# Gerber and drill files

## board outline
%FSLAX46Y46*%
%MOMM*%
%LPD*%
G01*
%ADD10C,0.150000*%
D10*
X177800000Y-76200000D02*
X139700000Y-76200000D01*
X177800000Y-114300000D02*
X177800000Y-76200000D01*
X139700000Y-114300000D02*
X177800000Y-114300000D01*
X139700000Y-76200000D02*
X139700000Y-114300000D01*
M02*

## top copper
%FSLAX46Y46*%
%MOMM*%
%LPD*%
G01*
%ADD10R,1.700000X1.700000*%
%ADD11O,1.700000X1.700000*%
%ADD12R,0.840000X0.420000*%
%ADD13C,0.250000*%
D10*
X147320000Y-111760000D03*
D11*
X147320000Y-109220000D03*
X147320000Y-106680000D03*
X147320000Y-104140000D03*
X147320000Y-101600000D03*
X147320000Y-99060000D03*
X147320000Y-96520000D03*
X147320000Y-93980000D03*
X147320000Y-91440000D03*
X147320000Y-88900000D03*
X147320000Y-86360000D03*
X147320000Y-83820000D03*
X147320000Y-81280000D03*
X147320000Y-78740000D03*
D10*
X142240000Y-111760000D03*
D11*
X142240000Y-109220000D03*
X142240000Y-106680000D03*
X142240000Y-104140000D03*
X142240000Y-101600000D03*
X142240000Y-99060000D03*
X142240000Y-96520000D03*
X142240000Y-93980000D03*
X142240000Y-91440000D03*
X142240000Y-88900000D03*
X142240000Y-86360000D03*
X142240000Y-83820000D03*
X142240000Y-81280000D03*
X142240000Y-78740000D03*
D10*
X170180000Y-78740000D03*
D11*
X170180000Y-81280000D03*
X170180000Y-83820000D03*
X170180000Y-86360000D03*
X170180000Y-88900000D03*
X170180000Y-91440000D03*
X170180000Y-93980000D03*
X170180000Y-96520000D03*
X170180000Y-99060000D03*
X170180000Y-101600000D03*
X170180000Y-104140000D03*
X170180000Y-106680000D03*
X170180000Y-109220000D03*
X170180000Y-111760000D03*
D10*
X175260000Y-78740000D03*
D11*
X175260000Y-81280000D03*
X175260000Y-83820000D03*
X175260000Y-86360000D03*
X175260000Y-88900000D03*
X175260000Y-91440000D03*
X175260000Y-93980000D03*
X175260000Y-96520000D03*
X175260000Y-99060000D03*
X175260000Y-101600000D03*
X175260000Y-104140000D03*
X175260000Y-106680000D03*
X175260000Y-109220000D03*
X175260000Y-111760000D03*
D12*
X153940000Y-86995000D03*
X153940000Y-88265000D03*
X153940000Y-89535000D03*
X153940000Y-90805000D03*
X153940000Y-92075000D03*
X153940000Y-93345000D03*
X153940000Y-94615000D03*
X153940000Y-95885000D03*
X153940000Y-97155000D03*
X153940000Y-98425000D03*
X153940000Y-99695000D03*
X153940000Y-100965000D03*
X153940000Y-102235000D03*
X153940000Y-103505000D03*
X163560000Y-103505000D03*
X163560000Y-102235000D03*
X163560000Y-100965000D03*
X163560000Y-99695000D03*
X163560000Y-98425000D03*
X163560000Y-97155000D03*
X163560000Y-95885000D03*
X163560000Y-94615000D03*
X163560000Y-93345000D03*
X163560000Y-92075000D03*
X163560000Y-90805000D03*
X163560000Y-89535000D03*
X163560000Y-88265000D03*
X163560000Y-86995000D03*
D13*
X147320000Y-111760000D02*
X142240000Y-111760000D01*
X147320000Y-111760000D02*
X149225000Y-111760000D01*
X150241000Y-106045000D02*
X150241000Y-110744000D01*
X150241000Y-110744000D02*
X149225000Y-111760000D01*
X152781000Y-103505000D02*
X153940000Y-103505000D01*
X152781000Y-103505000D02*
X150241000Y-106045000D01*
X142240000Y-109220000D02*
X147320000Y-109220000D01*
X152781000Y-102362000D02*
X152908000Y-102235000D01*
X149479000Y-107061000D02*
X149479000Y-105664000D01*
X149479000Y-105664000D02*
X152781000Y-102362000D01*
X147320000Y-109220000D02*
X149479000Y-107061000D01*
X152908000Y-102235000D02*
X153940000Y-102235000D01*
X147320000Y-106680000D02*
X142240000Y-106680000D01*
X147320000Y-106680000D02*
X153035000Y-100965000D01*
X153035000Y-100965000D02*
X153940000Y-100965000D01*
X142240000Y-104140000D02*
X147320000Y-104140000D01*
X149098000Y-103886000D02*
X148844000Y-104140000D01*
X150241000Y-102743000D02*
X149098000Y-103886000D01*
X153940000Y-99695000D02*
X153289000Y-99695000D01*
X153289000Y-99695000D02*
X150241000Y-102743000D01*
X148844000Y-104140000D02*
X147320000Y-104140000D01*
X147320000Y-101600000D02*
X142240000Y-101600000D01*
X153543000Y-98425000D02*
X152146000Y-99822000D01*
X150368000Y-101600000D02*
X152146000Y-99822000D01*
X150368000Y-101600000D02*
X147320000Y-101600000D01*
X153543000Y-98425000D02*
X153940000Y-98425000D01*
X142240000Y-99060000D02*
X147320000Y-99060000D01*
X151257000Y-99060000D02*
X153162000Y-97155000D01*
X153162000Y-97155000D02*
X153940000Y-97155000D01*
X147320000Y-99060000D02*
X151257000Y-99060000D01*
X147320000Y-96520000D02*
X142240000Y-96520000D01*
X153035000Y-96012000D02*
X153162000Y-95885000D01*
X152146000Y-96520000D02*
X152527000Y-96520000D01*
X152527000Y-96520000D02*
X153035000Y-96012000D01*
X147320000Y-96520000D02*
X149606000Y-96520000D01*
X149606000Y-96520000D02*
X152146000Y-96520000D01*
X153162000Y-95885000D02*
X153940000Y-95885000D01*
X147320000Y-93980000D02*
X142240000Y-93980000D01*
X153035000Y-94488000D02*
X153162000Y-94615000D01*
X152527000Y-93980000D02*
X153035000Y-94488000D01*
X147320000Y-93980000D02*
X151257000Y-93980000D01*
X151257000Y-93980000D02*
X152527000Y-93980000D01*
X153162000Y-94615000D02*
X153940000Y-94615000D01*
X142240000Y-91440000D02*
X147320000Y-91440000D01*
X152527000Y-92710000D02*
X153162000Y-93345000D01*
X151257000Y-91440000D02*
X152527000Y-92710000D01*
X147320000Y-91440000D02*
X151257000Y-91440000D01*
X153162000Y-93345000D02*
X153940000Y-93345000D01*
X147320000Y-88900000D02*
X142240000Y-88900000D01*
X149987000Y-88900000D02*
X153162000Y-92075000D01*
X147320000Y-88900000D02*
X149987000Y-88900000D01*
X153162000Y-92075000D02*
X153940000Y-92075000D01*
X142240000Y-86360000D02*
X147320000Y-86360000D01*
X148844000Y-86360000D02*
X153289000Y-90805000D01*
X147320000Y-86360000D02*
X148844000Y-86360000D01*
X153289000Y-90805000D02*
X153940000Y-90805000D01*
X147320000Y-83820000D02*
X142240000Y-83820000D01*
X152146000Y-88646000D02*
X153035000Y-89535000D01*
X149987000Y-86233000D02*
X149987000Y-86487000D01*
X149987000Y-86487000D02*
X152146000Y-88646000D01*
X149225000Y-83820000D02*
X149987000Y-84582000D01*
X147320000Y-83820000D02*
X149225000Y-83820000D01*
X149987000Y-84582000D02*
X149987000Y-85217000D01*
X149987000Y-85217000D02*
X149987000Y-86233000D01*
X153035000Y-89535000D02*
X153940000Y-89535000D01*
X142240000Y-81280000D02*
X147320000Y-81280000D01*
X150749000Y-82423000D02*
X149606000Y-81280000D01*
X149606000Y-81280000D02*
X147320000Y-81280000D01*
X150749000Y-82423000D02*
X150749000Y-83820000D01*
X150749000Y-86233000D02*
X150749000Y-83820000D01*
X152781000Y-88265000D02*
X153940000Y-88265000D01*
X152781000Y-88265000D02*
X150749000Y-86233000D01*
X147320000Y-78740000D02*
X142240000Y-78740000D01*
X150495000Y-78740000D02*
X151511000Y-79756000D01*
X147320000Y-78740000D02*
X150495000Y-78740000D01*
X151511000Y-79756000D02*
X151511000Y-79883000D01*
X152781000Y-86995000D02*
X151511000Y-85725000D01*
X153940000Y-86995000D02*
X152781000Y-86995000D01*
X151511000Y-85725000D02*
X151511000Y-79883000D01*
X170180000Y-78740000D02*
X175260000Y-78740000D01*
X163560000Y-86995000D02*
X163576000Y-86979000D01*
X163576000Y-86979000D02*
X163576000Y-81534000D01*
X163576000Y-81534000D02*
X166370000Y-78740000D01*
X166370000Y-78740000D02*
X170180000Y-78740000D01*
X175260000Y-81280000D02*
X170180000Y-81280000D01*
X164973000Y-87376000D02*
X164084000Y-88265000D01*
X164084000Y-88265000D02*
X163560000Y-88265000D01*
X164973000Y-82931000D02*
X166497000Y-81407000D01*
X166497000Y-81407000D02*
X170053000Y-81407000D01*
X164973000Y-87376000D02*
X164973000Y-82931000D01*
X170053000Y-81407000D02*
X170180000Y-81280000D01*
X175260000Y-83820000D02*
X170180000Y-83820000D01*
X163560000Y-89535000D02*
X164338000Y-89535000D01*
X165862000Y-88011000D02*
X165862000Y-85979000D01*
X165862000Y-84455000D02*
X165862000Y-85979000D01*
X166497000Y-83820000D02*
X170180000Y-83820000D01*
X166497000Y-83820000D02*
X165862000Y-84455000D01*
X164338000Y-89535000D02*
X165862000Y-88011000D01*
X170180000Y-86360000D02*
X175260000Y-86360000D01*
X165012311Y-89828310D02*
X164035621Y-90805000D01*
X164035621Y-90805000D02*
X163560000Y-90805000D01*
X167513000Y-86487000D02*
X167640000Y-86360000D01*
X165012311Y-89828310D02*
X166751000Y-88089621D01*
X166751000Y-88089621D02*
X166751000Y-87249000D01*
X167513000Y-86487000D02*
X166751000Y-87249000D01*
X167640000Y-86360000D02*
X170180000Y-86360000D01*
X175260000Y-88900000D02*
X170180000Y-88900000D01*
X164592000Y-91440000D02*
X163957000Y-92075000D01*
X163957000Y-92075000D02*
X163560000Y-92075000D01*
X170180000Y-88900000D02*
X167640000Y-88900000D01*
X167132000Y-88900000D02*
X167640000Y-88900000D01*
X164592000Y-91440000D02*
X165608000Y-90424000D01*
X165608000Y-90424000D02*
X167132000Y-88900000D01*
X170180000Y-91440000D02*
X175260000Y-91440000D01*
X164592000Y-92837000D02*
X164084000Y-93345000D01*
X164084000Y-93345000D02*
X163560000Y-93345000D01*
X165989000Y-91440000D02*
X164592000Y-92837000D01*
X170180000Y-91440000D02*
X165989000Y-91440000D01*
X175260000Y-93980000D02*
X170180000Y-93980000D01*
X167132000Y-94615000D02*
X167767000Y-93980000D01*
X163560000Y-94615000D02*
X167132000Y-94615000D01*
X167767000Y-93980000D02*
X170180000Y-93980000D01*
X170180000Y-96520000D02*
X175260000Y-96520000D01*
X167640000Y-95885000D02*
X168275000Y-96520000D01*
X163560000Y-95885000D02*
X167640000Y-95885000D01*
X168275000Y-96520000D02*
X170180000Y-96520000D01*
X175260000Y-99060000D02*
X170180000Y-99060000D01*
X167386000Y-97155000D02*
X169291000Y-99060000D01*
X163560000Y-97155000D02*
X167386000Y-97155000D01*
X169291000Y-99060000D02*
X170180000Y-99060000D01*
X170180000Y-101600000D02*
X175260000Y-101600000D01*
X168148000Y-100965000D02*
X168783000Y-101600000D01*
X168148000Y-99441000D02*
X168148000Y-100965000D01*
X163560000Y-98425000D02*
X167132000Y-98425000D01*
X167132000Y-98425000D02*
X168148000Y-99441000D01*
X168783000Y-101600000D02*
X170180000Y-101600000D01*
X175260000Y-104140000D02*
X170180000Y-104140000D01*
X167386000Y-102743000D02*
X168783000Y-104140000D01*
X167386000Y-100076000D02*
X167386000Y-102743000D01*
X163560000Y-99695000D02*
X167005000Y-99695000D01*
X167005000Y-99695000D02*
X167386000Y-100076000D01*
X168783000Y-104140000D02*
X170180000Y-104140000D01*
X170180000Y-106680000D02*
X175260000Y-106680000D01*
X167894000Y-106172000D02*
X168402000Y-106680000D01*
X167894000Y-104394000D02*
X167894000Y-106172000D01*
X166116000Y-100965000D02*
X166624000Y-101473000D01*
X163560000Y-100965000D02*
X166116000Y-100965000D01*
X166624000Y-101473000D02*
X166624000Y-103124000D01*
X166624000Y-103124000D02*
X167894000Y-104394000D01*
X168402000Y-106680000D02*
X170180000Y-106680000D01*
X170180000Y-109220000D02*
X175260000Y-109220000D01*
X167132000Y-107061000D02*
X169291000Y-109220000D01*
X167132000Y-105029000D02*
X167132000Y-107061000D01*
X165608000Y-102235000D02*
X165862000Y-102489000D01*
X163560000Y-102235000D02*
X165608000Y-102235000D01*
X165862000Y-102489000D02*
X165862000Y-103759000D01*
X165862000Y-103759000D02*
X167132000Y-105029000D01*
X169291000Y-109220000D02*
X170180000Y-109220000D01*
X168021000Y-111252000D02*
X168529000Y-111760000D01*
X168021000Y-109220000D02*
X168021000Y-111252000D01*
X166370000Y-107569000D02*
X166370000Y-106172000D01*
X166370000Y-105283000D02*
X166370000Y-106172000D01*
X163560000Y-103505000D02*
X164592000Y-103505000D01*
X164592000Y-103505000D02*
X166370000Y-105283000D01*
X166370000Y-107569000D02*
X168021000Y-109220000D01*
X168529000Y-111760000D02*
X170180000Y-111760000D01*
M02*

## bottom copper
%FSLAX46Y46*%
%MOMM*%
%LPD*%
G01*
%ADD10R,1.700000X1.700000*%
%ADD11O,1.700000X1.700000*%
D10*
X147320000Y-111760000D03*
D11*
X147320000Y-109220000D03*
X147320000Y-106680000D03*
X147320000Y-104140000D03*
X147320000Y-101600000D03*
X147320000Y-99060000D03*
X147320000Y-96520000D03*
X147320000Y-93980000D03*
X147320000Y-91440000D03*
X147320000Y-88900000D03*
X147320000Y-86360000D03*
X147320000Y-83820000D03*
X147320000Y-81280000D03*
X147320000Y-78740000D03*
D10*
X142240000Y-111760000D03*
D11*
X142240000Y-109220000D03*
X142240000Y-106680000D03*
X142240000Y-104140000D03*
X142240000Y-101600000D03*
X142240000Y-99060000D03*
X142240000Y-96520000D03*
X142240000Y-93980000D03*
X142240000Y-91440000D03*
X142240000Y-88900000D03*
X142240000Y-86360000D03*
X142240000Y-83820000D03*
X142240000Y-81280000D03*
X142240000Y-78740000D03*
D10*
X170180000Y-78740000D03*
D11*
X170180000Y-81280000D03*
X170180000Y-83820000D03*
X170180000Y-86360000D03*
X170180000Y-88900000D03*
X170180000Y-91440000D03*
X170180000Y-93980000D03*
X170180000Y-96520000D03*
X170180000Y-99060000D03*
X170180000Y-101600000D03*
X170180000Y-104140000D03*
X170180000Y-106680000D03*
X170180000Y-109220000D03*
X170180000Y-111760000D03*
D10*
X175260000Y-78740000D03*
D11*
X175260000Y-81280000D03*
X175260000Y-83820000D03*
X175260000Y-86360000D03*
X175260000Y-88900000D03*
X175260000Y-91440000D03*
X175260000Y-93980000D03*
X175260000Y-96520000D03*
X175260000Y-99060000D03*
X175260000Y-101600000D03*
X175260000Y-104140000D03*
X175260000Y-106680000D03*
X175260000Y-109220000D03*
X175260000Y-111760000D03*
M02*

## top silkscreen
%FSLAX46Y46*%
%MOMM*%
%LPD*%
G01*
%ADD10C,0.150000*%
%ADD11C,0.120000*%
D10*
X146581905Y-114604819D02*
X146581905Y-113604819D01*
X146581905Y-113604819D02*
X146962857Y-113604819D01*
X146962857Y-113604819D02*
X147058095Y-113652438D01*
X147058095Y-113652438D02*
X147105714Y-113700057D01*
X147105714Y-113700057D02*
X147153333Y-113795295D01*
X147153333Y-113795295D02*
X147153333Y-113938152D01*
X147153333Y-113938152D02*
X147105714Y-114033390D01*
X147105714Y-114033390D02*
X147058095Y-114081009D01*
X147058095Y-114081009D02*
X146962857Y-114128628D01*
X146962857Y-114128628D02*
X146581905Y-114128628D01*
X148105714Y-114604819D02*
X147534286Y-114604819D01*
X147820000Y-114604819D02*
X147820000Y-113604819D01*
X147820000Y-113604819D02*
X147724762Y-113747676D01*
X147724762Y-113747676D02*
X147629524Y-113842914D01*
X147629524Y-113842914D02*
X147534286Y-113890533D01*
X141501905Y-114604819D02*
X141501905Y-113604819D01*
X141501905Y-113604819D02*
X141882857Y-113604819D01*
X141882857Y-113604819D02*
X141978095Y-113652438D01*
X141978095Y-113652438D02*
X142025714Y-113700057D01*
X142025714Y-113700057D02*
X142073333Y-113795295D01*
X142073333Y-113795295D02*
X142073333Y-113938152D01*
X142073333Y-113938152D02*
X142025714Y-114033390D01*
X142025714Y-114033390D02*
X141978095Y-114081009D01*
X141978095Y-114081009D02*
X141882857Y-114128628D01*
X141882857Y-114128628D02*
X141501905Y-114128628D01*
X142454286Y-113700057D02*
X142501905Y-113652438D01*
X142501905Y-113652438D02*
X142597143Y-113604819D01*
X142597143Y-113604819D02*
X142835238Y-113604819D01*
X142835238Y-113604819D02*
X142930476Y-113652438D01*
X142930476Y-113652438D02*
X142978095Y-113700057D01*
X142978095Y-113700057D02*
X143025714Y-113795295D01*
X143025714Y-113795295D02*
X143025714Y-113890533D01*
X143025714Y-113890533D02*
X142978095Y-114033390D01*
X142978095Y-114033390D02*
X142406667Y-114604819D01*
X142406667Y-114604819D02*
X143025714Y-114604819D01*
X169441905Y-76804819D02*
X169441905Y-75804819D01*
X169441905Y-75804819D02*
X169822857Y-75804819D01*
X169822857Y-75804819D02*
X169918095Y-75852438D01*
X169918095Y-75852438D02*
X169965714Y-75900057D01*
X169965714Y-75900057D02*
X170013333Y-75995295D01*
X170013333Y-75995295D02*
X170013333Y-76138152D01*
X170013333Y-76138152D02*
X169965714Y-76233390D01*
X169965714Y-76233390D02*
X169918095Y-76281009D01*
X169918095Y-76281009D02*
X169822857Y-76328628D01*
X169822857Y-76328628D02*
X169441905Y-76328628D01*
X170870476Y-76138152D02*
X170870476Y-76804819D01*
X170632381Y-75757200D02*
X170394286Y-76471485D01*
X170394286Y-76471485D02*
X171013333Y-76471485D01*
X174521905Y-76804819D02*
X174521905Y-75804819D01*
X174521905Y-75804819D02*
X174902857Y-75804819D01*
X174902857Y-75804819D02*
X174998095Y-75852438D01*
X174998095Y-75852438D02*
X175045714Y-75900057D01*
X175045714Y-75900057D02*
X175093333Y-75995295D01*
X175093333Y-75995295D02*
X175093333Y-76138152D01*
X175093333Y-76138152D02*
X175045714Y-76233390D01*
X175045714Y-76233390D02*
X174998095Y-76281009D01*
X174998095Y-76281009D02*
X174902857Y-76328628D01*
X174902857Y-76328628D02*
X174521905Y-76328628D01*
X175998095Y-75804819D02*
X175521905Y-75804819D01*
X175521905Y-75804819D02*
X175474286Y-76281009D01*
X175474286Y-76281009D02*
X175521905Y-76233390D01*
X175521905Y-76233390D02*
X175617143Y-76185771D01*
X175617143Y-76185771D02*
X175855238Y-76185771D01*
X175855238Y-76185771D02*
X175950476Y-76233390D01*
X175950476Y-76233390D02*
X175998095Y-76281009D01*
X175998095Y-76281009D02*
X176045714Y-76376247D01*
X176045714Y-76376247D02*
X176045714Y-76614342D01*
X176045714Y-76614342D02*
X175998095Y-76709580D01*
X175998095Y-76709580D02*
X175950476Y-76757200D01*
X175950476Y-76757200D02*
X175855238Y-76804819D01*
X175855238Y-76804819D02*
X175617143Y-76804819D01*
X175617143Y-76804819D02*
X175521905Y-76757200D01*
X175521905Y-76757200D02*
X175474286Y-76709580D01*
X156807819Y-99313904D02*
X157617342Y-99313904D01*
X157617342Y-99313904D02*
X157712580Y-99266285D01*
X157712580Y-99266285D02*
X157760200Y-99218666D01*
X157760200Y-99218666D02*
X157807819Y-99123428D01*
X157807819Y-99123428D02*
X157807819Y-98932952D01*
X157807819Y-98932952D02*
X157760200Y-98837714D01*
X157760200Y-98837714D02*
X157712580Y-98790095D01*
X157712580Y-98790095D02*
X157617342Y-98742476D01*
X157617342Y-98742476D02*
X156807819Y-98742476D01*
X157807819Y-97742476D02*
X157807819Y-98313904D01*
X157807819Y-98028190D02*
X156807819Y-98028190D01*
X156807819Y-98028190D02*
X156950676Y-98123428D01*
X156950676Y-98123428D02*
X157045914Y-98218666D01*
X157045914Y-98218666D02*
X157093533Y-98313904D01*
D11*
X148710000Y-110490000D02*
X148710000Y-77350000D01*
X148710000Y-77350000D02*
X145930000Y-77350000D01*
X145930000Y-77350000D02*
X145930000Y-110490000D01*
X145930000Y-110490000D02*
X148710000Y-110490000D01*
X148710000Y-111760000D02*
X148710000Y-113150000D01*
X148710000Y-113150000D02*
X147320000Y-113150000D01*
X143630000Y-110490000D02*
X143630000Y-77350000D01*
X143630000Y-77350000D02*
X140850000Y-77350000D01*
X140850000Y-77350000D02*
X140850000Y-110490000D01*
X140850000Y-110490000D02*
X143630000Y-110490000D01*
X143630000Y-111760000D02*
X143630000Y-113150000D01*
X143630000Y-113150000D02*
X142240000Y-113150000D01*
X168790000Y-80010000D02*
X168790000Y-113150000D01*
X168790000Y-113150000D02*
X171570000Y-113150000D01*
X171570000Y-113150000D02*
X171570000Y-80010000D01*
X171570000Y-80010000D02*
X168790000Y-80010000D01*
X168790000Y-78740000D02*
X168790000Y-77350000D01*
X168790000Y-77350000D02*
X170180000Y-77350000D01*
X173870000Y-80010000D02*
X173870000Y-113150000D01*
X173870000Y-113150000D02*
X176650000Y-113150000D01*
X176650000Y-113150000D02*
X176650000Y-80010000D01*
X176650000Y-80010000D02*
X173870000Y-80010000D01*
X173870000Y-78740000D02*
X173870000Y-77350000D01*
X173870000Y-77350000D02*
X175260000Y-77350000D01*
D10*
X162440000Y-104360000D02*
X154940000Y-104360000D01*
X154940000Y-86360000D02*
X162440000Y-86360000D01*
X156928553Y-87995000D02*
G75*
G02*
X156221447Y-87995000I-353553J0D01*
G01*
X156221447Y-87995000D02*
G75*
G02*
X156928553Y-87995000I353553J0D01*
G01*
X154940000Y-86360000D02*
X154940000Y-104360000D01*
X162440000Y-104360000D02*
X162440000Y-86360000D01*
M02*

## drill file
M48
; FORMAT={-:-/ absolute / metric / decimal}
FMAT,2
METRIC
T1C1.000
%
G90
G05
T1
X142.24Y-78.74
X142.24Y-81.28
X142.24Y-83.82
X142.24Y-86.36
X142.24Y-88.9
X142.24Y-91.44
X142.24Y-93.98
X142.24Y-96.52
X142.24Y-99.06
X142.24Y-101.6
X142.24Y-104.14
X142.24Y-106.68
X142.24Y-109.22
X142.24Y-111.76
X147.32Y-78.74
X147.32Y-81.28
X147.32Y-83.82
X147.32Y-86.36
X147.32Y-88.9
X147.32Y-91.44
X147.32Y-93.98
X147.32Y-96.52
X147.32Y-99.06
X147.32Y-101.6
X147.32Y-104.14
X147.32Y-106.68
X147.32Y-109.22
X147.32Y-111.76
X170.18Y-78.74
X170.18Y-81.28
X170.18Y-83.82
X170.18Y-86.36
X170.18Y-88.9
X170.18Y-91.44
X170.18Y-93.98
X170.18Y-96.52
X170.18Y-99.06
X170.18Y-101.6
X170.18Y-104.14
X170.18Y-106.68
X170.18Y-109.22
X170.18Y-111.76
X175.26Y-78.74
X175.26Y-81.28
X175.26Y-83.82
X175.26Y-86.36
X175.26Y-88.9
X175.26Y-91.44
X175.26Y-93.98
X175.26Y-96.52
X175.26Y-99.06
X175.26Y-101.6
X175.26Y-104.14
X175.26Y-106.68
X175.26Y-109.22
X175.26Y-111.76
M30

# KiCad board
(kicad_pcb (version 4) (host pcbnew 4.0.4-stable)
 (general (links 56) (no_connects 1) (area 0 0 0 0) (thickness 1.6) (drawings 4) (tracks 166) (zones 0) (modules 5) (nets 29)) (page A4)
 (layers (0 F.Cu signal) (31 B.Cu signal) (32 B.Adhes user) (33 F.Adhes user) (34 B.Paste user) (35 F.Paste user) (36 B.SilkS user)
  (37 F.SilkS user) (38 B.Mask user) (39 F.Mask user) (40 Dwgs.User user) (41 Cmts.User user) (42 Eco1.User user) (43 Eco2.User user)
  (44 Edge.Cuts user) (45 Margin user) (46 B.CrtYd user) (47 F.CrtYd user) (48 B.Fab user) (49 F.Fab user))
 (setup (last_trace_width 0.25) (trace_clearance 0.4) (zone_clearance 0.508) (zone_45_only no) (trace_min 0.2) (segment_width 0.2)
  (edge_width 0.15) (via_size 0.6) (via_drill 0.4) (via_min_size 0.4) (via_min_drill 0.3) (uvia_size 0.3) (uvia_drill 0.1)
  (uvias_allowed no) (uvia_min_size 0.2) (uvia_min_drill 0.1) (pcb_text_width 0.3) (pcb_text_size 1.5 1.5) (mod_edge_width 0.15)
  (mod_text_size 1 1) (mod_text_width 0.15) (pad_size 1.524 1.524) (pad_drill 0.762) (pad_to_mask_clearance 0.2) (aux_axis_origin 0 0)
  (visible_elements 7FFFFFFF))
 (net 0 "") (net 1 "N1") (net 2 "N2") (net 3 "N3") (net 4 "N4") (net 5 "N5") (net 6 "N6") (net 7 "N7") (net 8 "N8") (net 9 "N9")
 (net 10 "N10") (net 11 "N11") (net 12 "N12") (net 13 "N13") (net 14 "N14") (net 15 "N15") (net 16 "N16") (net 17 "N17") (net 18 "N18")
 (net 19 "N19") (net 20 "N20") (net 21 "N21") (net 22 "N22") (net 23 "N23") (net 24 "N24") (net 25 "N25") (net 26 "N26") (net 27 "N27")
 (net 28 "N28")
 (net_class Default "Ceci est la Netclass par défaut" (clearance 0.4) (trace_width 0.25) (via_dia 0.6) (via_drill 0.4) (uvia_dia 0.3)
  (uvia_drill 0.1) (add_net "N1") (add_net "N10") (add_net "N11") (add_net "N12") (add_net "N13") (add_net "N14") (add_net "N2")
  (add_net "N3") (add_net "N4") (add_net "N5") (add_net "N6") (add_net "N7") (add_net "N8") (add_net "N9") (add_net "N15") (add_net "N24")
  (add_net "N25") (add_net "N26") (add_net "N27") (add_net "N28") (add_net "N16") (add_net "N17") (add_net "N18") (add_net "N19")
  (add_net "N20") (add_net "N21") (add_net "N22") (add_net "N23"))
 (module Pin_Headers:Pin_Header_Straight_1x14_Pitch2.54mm (layer F.Cu) (at 147.32 111.76 180)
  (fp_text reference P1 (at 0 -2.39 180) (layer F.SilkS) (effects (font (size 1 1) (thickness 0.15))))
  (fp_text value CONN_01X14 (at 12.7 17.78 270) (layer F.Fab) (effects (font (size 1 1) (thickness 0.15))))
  (fp_line (start -1.39 1.27) (end -1.39 34.41) (layer F.SilkS) (width 0.12))
  (fp_line (start -1.39 34.41) (end 1.39 34.41) (layer F.SilkS) (width 0.12))
  (fp_line (start 1.39 34.41) (end 1.39 1.27) (layer F.SilkS) (width 0.12))
  (fp_line (start 1.39 1.27) (end -1.39 1.27) (layer F.SilkS) (width 0.12))
  (fp_line (start -1.39 0) (end -1.39 -1.39) (layer F.SilkS) (width 0.12))
  (fp_line (start -1.39 -1.39) (end 0 -1.39) (layer F.SilkS) (width 0.12))
  (pad 1 thru_hole rect (at 0 0 180) (size 1.7 1.7) (drill 1) (layers *.Cu *.Mask) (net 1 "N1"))
  (pad 2 thru_hole oval (at 0 2.54 180) (size 1.7 1.7) (drill 1) (layers *.Cu *.Mask) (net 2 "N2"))
  (pad 3 thru_hole oval (at 0 5.08 180) (size 1.7 1.7) (drill 1) (layers *.Cu *.Mask) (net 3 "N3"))
  (pad 4 thru_hole oval (at 0 7.62 180) (size 1.7 1.7) (drill 1) (layers *.Cu *.Mask) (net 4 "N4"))
  (pad 5 thru_hole oval (at 0 10.16 180) (size 1.7 1.7) (drill 1) (layers *.Cu *.Mask) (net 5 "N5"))
  (pad 6 thru_hole oval (at 0 12.7 180) (size 1.7 1.7) (drill 1) (layers *.Cu *.Mask) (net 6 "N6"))
  (pad 7 thru_hole oval (at 0 15.24 180) (size 1.7 1.7) (drill 1) (layers *.Cu *.Mask) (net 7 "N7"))
  (pad 8 thru_hole oval (at 0 17.78 180) (size 1.7 1.7) (drill 1) (layers *.Cu *.Mask) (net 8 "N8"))
  (pad 9 thru_hole oval (at 0 20.32 180) (size 1.7 1.7) (drill 1) (layers *.Cu *.Mask) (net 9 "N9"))
  (pad 10 thru_hole oval (at 0 22.86 180) (size 1.7 1.7) (drill 1) (layers *.Cu *.Mask) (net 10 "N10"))
  (pad 11 thru_hole oval (at 0 25.4 180) (size 1.7 1.7) (drill 1) (layers *.Cu *.Mask) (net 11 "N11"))
  (pad 12 thru_hole oval (at 0 27.94 180) (size 1.7 1.7) (drill 1) (layers *.Cu *.Mask) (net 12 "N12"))
  (pad 13 thru_hole oval (at 0 30.48 180) (size 1.7 1.7) (drill 1) (layers *.Cu *.Mask) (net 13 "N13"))
  (pad 14 thru_hole oval (at 0 33.02 180) (size 1.7 1.7) (drill 1) (layers *.Cu *.Mask) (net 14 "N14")))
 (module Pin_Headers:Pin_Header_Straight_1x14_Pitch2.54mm (layer F.Cu) (at 142.24 111.76 180)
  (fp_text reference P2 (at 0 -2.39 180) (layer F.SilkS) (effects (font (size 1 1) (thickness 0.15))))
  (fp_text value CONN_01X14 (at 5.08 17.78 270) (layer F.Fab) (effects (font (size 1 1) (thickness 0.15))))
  (fp_line (start -1.39 1.27) (end -1.39 34.41) (layer F.SilkS) (width 0.12))
  (fp_line (start -1.39 34.41) (end 1.39 34.41) (layer F.SilkS) (width 0.12))
  (fp_line (start 1.39 34.41) (end 1.39 1.27) (layer F.SilkS) (width 0.12))
  (fp_line (start 1.39 1.27) (end -1.39 1.27) (layer F.SilkS) (width 0.12))
  (fp_line (start -1.39 0) (end -1.39 -1.39) (layer F.SilkS) (width 0.12))
  (fp_line (start -1.39 -1.39) (end 0 -1.39) (layer F.SilkS) (width 0.12))
  (pad 1 thru_hole rect (at 0 0 180) (size 1.7 1.7) (drill 1) (layers *.Cu *.Mask) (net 1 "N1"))
  (pad 2 thru_hole oval (at 0 2.54 180) (size 1.7 1.7) (drill 1) (layers *.Cu *.Mask) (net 2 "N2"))
  (pad 3 thru_hole oval (at 0 5.08 180) (size 1.7 1.7) (drill 1) (layers *.Cu *.Mask) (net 3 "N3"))
  (pad 4 thru_hole oval (at 0 7.62 180) (size 1.7 1.7) (drill 1) (layers *.Cu *.Mask) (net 4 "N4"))
  (pad 5 thru_hole oval (at 0 10.16 180) (size 1.7 1.7) (drill 1) (layers *.Cu *.Mask) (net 5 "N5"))
  (pad 6 thru_hole oval (at 0 12.7 180) (size 1.7 1.7) (drill 1) (layers *.Cu *.Mask) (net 6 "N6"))
  (pad 7 thru_hole oval (at 0 15.24 180) (size 1.7 1.7) (drill 1) (layers *.Cu *.Mask) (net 7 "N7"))
  (pad 8 thru_hole oval (at 0 17.78 180) (size 1.7 1.7) (drill 1) (layers *.Cu *.Mask) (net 8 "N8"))
  (pad 9 thru_hole oval (at 0 20.32 180) (size 1.7 1.7) (drill 1) (layers *.Cu *.Mask) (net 9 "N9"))
  (pad 10 thru_hole oval (at 0 22.86 180) (size 1.7 1.7) (drill 1) (layers *.Cu *.Mask) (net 10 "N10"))
  (pad 11 thru_hole oval (at 0 25.4 180) (size 1.7 1.7) (drill 1) (layers *.Cu *.Mask) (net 11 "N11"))
  (pad 12 thru_hole oval (at 0 27.94 180) (size 1.7 1.7) (drill 1) (layers *.Cu *.Mask) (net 12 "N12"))
  (pad 13 thru_hole oval (at 0 30.48 180) (size 1.7 1.7) (drill 1) (layers *.Cu *.Mask) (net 13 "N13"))
  (pad 14 thru_hole oval (at 0 33.02 180) (size 1.7 1.7) (drill 1) (layers *.Cu *.Mask) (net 14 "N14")))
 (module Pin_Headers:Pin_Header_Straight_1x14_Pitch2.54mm (layer F.Cu) (at 170.18 78.74)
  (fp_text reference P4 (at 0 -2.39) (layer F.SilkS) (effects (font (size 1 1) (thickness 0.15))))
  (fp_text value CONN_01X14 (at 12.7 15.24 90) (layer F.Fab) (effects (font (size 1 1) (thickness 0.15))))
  (fp_line (start -1.39 1.27) (end -1.39 34.41) (layer F.SilkS) (width 0.12))
  (fp_line (start -1.39 34.41) (end 1.39 34.41) (layer F.SilkS) (width 0.12))
  (fp_line (start 1.39 34.41) (end 1.39 1.27) (layer F.SilkS) (width 0.12))
  (fp_line (start 1.39 1.27) (end -1.39 1.27) (layer F.SilkS) (width 0.12))
  (fp_line (start -1.39 0) (end -1.39 -1.39) (layer F.SilkS) (width 0.12))
  (fp_line (start -1.39 -1.39) (end 0 -1.39) (layer F.SilkS) (width 0.12))
  (pad 1 thru_hole rect (at 0 0) (size 1.7 1.7) (drill 1) (layers *.Cu *.Mask) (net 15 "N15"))
  (pad 2 thru_hole oval (at 0 2.54) (size 1.7 1.7) (drill 1) (layers *.Cu *.Mask) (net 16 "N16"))
  (pad 3 thru_hole oval (at 0 5.08) (size 1.7 1.7) (drill 1) (layers *.Cu *.Mask) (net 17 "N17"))
  (pad 4 thru_hole oval (at 0 7.62) (size 1.7 1.7) (drill 1) (layers *.Cu *.Mask) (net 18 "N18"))
  (pad 5 thru_hole oval (at 0 10.16) (size 1.7 1.7) (drill 1) (layers *.Cu *.Mask) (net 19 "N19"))
  (pad 6 thru_hole oval (at 0 12.7) (size 1.7 1.7) (drill 1) (layers *.Cu *.Mask) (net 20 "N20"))
  (pad 7 thru_hole oval (at 0 15.24) (size 1.7 1.7) (drill 1) (layers *.Cu *.Mask) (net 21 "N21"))
  (pad 8 thru_hole oval (at 0 17.78) (size 1.7 1.7) (drill 1) (layers *.Cu *.Mask) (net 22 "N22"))
  (pad 9 thru_hole oval (at 0 20.32) (size 1.7 1.7) (drill 1) (layers *.Cu *.Mask) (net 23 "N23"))
  (pad 10 thru_hole oval (at 0 22.86) (size 1.7 1.7) (drill 1) (layers *.Cu *.Mask) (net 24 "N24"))
  (pad 11 thru_hole oval (at 0 25.4) (size 1.7 1.7) (drill 1) (layers *.Cu *.Mask) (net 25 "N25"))
  (pad 12 thru_hole oval (at 0 27.94) (size 1.7 1.7) (drill 1) (layers *.Cu *.Mask) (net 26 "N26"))
  (pad 13 thru_hole oval (at 0 30.48) (size 1.7 1.7) (drill 1) (layers *.Cu *.Mask) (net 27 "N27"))
  (pad 14 thru_hole oval (at 0 33.02) (size 1.7 1.7) (drill 1) (layers *.Cu *.Mask) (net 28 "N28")))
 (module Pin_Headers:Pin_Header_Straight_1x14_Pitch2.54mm (layer F.Cu) (at 175.26 78.74)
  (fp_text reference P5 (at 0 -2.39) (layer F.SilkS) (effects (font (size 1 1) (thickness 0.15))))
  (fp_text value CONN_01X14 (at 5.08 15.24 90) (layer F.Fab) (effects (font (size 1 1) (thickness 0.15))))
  (fp_line (start -1.39 1.27) (end -1.39 34.41) (layer F.SilkS) (width 0.12))
  (fp_line (start -1.39 34.41) (end 1.39 34.41) (layer F.SilkS) (width 0.12))
  (fp_line (start 1.39 34.41) (end 1.39 1.27) (layer F.SilkS) (width 0.12))
  (fp_line (start 1.39 1.27) (end -1.39 1.27) (layer F.SilkS) (width 0.12))
  (fp_line (start -1.39 0) (end -1.39 -1.39) (layer F.SilkS) (width 0.12))
  (fp_line (start -1.39 -1.39) (end 0 -1.39) (layer F.SilkS) (width 0.12))
  (pad 1 thru_hole rect (at 0 0) (size 1.7 1.7) (drill 1) (layers *.Cu *.Mask) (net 15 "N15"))
  (pad 2 thru_hole oval (at 0 2.54) (size 1.7 1.7) (drill 1) (layers *.Cu *.Mask) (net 16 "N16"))
  (pad 3 thru_hole oval (at 0 5.08) (size 1.7 1.7) (drill 1) (layers *.Cu *.Mask) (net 17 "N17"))
  (pad 4 thru_hole oval (at 0 7.62) (size 1.7 1.7) (drill 1) (layers *.Cu *.Mask) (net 18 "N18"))
  (pad 5 thru_hole oval (at 0 10.16) (size 1.7 1.7) (drill 1) (layers *.Cu *.Mask) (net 19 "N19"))
  (pad 6 thru_hole oval (at 0 12.7) (size 1.7 1.7) (drill 1) (layers *.Cu *.Mask) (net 20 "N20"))
  (pad 7 thru_hole oval (at 0 15.24) (size 1.7 1.7) (drill 1) (layers *.Cu *.Mask) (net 21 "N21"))
  (pad 8 thru_hole oval (at 0 17.78) (size 1.7 1.7) (drill 1) (layers *.Cu *.Mask) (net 22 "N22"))
  (pad 9 thru_hole oval (at 0 20.32) (size 1.7 1.7) (drill 1) (layers *.Cu *.Mask) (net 23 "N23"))
  (pad 10 thru_hole oval (at 0 22.86) (size 1.7 1.7) (drill 1) (layers *.Cu *.Mask) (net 24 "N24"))
  (pad 11 thru_hole oval (at 0 25.4) (size 1.7 1.7) (drill 1) (layers *.Cu *.Mask) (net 25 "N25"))
  (pad 12 thru_hole oval (at 0 27.94) (size 1.7 1.7) (drill 1) (layers *.Cu *.Mask) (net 26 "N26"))
  (pad 13 thru_hole oval (at 0 30.48) (size 1.7 1.7) (drill 1) (layers *.Cu *.Mask) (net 27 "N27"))
  (pad 14 thru_hole oval (at 0 33.02) (size 1.7 1.7) (drill 1) (layers *.Cu *.Mask) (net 28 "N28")))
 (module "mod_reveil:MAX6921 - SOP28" (layer F.Cu) (at 154.94 86.36 270)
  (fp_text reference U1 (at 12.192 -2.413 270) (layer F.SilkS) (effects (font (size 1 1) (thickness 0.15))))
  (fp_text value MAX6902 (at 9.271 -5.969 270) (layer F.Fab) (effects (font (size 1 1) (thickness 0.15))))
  (fp_line (start 18 -7.5) (end 18 0) (layer F.SilkS) (width 0.15))
  (fp_line (start 0 0) (end 0 -7.5) (layer F.SilkS) (width 0.15))
  (fp_circle (center 1.635 -1.635) (end 1.885 -1.385) (layer F.SilkS) (width 0.15))
  (fp_line (start 0 0) (end 18 0) (layer F.SilkS) (width 0.15))
  (fp_line (start 18 -7.5) (end 0 -7.5) (layer F.SilkS) (width 0.15))
  (pad 1 smd rect (at 0.635 1 270) (size 0.42 0.84) (layers F.Cu F.Paste F.Mask) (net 14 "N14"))
  (pad 2 smd rect (at 1.905 1 270) (size 0.42 0.84) (layers F.Cu F.Paste F.Mask) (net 13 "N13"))
  (pad 3 smd rect (at 3.175 1 270) (size 0.42 0.84) (layers F.Cu F.Paste F.Mask) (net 12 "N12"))
  (pad 4 smd rect (at 4.445 1 270) (size 0.42 0.84) (layers F.Cu F.Paste F.Mask) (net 11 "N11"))
  (pad 5 smd rect (at 5.715 1 270) (size 0.42 0.84) (layers F.Cu F.Paste F.Mask) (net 10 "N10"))
  (pad 6 smd rect (at 6.985 1 270) (size 0.42 0.84) (layers F.Cu F.Paste F.Mask) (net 9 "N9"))
  (pad 7 smd rect (at 8.255 1 270) (size 0.42 0.84) (layers F.Cu F.Paste F.Mask) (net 8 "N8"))
  (pad 8 smd rect (at 9.525 1 270) (size 0.42 0.84) (layers F.Cu F.Paste F.Mask) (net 7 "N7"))
  (pad 9 smd rect (at 10.795 1 270) (size 0.42 0.84) (layers F.Cu F.Paste F.Mask) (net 6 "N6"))
  (pad 10 smd rect (at 12.065 1 270) (size 0.42 0.84) (layers F.Cu F.Paste F.Mask) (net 5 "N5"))
  (pad 11 smd rect (at 13.335 1 270) (size 0.42 0.84) (layers F.Cu F.Paste F.Mask) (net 4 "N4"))
  (pad 12 smd rect (at 14.605 1 270) (size 0.42 0.84) (layers F.Cu F.Paste F.Mask) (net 3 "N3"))
  (pad 13 smd rect (at 15.875 1 270) (size 0.42 0.84) (layers F.Cu F.Paste F.Mask) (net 2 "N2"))
  (pad 14 smd rect (at 17.145 1 270) (size 0.42 0.84) (layers F.Cu F.Paste F.Mask) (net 1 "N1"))
  (pad 15 smd rect (at 17.145 -8.62 270) (size 0.42 0.84) (layers F.Cu F.Paste F.Mask) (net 28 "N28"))
  (pad 16 smd rect (at 15.875 -8.62 270) (size 0.42 0.84) (layers F.Cu F.Paste F.Mask) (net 27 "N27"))
  (pad 17 smd rect (at 14.605 -8.62 270) (size 0.42 0.84) (layers F.Cu F.Paste F.Mask) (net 26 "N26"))
  (pad 18 smd rect (at 13.335 -8.62 270) (size 0.42 0.84) (layers F.Cu F.Paste F.Mask) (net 25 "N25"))
  (pad 19 smd rect (at 12.065 -8.62 270) (size 0.42 0.84) (layers F.Cu F.Paste F.Mask) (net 24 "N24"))
  (pad 20 smd rect (at 10.795 -8.62 270) (size 0.42 0.84) (layers F.Cu F.Paste F.Mask) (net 23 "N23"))
  (pad 21 smd rect (at 9.525 -8.62 270) (size 0.42 0.84) (layers F.Cu F.Paste F.Mask) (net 22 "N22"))
  (pad 22 smd rect (at 8.255 -8.62 270) (size 0.42 0.84) (layers F.Cu F.Paste F.Mask) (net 21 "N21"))
  (pad 23 smd rect (at 6.985 -8.62 270) (size 0.42 0.84) (layers F.Cu F.Paste F.Mask) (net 20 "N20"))
  (pad 24 smd rect (at 5.715 -8.62 270) (size 0.42 0.84) (layers F.Cu F.Paste F.Mask) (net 19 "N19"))
  (pad 25 smd rect (at 4.445 -8.62 270) (size 0.42 0.84) (layers F.Cu F.Paste F.Mask) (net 18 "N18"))
  (pad 26 smd rect (at 3.175 -8.62 270) (size 0.42 0.84) (layers F.Cu F.Paste F.Mask) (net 17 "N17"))
  (pad 27 smd rect (at 1.905 -8.62 270) (size 0.42 0.84) (layers F.Cu F.Paste F.Mask) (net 16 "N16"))
  (pad 28 smd rect (at 0.635 -8.62 270) (size 0.42 0.84) (layers F.Cu F.Paste F.Mask) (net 15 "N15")))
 (gr_line (start 177.8 76.2) (end 139.7 76.2) (angle 90) (layer Edge.Cuts) (width 0.15))
 (gr_line (start 177.8 114.3) (end 177.8 76.2) (angle 90) (layer Edge.Cuts) (width 0.15))
 (gr_line (start 139.7 114.3) (end 177.8 114.3) (angle 90) (layer Edge.Cuts) (width 0.15))
 (gr_line (start 139.7 76.2) (end 139.7 114.3) (angle 90) (layer Edge.Cuts) (width 0.15))
 (segment (start 147.32 111.76) (end 142.24 111.76) (width 0.25) (layer F.Cu) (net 1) (status C00000))
 (segment (start 147.32 111.76) (end 149.225 111.76) (width 0.25) (layer F.Cu) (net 1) (status 400000))
 (segment (start 150.241 106.045) (end 150.241 110.744) (width 0.25) (layer F.Cu) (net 1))
 (segment (start 150.241 110.744) (end 149.225 111.76) (width 0.25) (layer F.Cu) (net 1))
 (segment (start 152.781 103.505) (end 153.94 103.505) (width 0.25) (layer F.Cu) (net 1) (status 800000))
 (segment (start 152.781 103.505) (end 150.241 106.045) (width 0.25) (layer F.Cu) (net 1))
 (segment (start 142.24 109.22) (end 147.32 109.22) (width 0.25) (layer F.Cu) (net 2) (status C00000))
 (segment (start 152.781 102.362) (end 152.908 102.235) (width 0.25) (layer F.Cu) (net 2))
 (segment (start 149.479 107.061) (end 149.479 105.664) (width 0.25) (layer F.Cu) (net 2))
 (segment (start 149.479 105.664) (end 152.781 102.362) (width 0.25) (layer F.Cu) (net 2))
 (segment (start 147.32 109.22) (end 149.479 107.061) (width 0.25) (layer F.Cu) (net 2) (status 400000))
 (segment (start 152.908 102.235) (end 153.94 102.235) (width 0.25) (layer F.Cu) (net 2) (status 800000))
 (segment (start 147.32 106.68) (end 142.24 106.68) (width 0.25) (layer F.Cu) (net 3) (status C00000))
 (segment (start 147.32 106.68) (end 153.035 100.965) (width 0.25) (layer F.Cu) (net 3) (status 400000))
 (segment (start 153.035 100.965) (end 153.94 100.965) (width 0.25) (layer F.Cu) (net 3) (status 800000))
 (segment (start 142.24 104.14) (end 147.32 104.14) (width 0.25) (layer F.Cu) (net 4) (status C00000))
 (segment (start 149.098 103.886) (end 148.844 104.14) (width 0.25) (layer F.Cu) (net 4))
 (segment (start 150.241 102.743) (end 149.098 103.886) (width 0.25) (layer F.Cu) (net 4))
 (segment (start 153.94 99.695) (end 153.289 99.695) (width 0.25) (layer F.Cu) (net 4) (status 400000))
 (segment (start 153.289 99.695) (end 150.241 102.743) (width 0.25) (layer F.Cu) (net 4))
 (segment (start 148.844 104.14) (end 147.32 104.14) (width 0.25) (layer F.Cu) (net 4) (status 800000))
 (segment (start 147.32 101.6) (end 142.24 101.6) (width 0.25) (layer F.Cu) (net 5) (status C00000))
 (segment (start 153.543 98.425) (end 152.146 99.822) (width 0.25) (layer F.Cu) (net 5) (status 400000))
 (segment (start 150.368 101.6) (end 152.146 99.822) (width 0.25) (layer F.Cu) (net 5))
 (segment (start 150.368 101.6) (end 147.32 101.6) (width 0.25) (layer F.Cu) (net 5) (status 800000))
 (segment (start 153.543 98.425) (end 153.94 98.425) (width 0.25) (layer F.Cu) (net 5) (status C00000))
 (segment (start 142.24 99.06) (end 147.32 99.06) (width 0.25) (layer F.Cu) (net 6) (status C00000))
 (segment (start 151.257 99.06) (end 153.162 97.155) (width 0.25) (layer F.Cu) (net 6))
 (segment (start 153.162 97.155) (end 153.94 97.155) (width 0.25) (layer F.Cu) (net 6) (status 800000))
 (segment (start 147.32 99.06) (end 151.257 99.06) (width 0.25) (layer F.Cu) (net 6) (status 400000))
 (segment (start 147.32 96.52) (end 142.24 96.52) (width 0.25) (layer F.Cu) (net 7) (status C00000))
 (segment (start 153.035 96.012) (end 153.162 95.885) (width 0.25) (layer F.Cu) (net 7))
 (segment (start 152.146 96.52) (end 152.527 96.52) (width 0.25) (layer F.Cu) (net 7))
 (segment (start 152.527 96.52) (end 153.035 96.012) (width 0.25) (layer F.Cu) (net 7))
 (segment (start 147.32 96.52) (end 149.606 96.52) (width 0.25) (layer F.Cu) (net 7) (status 400000))
 (segment (start 149.606 96.52) (end 152.146 96.52) (width 0.25) (layer F.Cu) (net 7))
 (segment (start 153.162 95.885) (end 153.94 95.885) (width 0.25) (layer F.Cu) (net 7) (status 800000))
 (segment (start 147.32 93.98) (end 142.24 93.98) (width 0.25) (layer F.Cu) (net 8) (status C00000))
 (segment (start 153.035 94.488) (end 153.162 94.615) (width 0.25) (layer F.Cu) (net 8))
 (segment (start 152.527 93.98) (end 153.035 94.488) (width 0.25) (layer F.Cu) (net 8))
 (segment (start 147.32 93.98) (end 151.257 93.98) (width 0.25) (layer F.Cu) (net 8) (status 400000))
 (segment (start 151.257 93.98) (end 152.527 93.98) (width 0.25) (layer F.Cu) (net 8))
 (segment (start 153.162 94.615) (end 153.94 94.615) (width 0.25) (layer F.Cu) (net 8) (status 800000))
 (segment (start 142.24 91.44) (end 147.32 91.44) (width 0.25) (layer F.Cu) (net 9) (status C00000))
 (segment (start 152.527 92.71) (end 153.162 93.345) (width 0.25) (layer F.Cu) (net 9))
 (segment (start 151.257 91.44) (end 152.527 92.71) (width 0.25) (layer F.Cu) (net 9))
 (segment (start 147.32 91.44) (end 151.257 91.44) (width 0.25) (layer F.Cu) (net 9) (status 400000))
 (segment (start 153.162 93.345) (end 153.94 93.345) (width 0.25) (layer F.Cu) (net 9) (status 800000))
 (segment (start 147.32 88.9) (end 142.24 88.9) (width 0.25) (layer F.Cu) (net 10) (status C00000))
 (segment (start 149.987 88.9) (end 153.162 92.075) (width 0.25) (layer F.Cu) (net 10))
 (segment (start 147.32 88.9) (end 149.987 88.9) (width 0.25) (layer F.Cu) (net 10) (status 400000))
 (segment (start 153.162 92.075) (end 153.94 92.075) (width 0.25) (layer F.Cu) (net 10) (status 800000))
 (segment (start 142.24 86.36) (end 147.32 86.36) (width 0.25) (layer F.Cu) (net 11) (status C00000))
 (segment (start 148.844 86.36) (end 153.289 90.805) (width 0.25) (layer F.Cu) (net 11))
 (segment (start 147.32 86.36) (end 148.844 86.36) (width 0.25) (layer F.Cu) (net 11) (status 400000))
 (segment (start 153.289 90.805) (end 153.94 90.805) (width 0.25) (layer F.Cu) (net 11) (status 800000))
 (segment (start 147.32 83.82) (end 142.24 83.82) (width 0.25) (layer F.Cu) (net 12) (status C00000))
 (segment (start 152.146 88.646) (end 153.035 89.535) (width 0.25) (layer F.Cu) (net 12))
 (segment (start 149.987 86.233) (end 149.987 86.487) (width 0.25) (layer F.Cu) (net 12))
 (segment (start 149.987 86.487) (end 152.146 88.646) (width 0.25) (layer F.Cu) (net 12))
 (segment (start 149.225 83.82) (end 149.987 84.582) (width 0.25) (layer F.Cu) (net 12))
 (segment (start 147.32 83.82) (end 149.225 83.82) (width 0.25) (layer F.Cu) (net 12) (status 400000))
 (segment (start 149.987 84.582) (end 149.987 85.217) (width 0.25) (layer F.Cu) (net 12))
 (segment (start 149.987 85.217) (end 149.987 86.233) (width 0.25) (layer F.Cu) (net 12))
 (segment (start 153.035 89.535) (end 153.94 89.535) (width 0.25) (layer F.Cu) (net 12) (status 800000))
 (segment (start 142.24 81.28) (end 147.32 81.28) (width 0.25) (layer F.Cu) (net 13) (status C00000))
 (segment (start 150.749 82.423) (end 149.606 81.28) (width 0.25) (layer F.Cu) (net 13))
 (segment (start 149.606 81.28) (end 147.32 81.28) (width 0.25) (layer F.Cu) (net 13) (status 800000))
 (segment (start 150.749 82.423) (end 150.749 83.82) (width 0.25) (layer F.Cu) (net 13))
 (segment (start 150.749 86.233) (end 150.749 83.82) (width 0.25) (layer F.Cu) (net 13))
 (segment (start 152.781 88.265) (end 153.94 88.265) (width 0.25) (layer F.Cu) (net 13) (status 800000))
 (segment (start 152.781 88.265) (end 150.749 86.233) (width 0.25) (layer F.Cu) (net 13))
 (segment (start 147.32 78.74) (end 142.24 78.74) (width 0.25) (layer F.Cu) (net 14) (status C00000))
 (segment (start 150.495 78.74) (end 151.511 79.756) (width 0.25) (layer F.Cu) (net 14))
 (segment (start 147.32 78.74) (end 150.495 78.74) (width 0.25) (layer F.Cu) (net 14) (status 400000))
 (segment (start 151.511 79.756) (end 151.511 79.883) (width 0.25) (layer F.Cu) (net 14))
 (segment (start 152.781 86.995) (end 151.511 85.725) (width 0.25) (layer F.Cu) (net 14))
 (segment (start 153.94 86.995) (end 152.781 86.995) (width 0.25) (layer F.Cu) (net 14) (status 400000))
 (segment (start 151.511 85.725) (end 151.511 79.883) (width 0.25) (layer F.Cu) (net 14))
 (segment (start 170.18 78.74) (end 175.26 78.74) (width 0.25) (layer F.Cu) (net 15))
 (segment (start 163.56 86.995) (end 163.576 86.979) (width 0.25) (layer F.Cu) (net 15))
 (segment (start 163.576 86.979) (end 163.576 81.534) (width 0.25) (layer F.Cu) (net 15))
 (segment (start 163.576 81.534) (end 166.37 78.74) (width 0.25) (layer F.Cu) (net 15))
 (segment (start 166.37 78.74) (end 170.18 78.74) (width 0.25) (layer F.Cu) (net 15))
 (segment (start 175.26 81.28) (end 170.18 81.28) (width 0.25) (layer F.Cu) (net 16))
 (segment (start 164.973 87.376) (end 164.084 88.265) (width 0.25) (layer F.Cu) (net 16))
 (segment (start 164.084 88.265) (end 163.56 88.265) (width 0.25) (layer F.Cu) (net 16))
 (segment (start 164.973 82.931) (end 166.497 81.407) (width 0.25) (layer F.Cu) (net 16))
 (segment (start 166.497 81.407) (end 170.053 81.407) (width 0.25) (layer F.Cu) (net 16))
 (segment (start 164.973 87.376) (end 164.973 82.931) (width 0.25) (layer F.Cu) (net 16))
 (segment (start 170.053 81.407) (end 170.18 81.28) (width 0.25) (layer F.Cu) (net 16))
 (segment (start 175.26 83.82) (end 170.18 83.82) (width 0.25) (layer F.Cu) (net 17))
 (segment (start 163.56 89.535) (end 164.338 89.535) (width 0.25) (layer F.Cu) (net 17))
 (segment (start 165.862 88.011) (end 165.862 85.979) (width 0.25) (layer F.Cu) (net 17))
 (segment (start 165.862 84.455) (end 165.862 85.979) (width 0.25) (layer F.Cu) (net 17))
 (segment (start 166.497 83.82) (end 170.18 83.82) (width 0.25) (layer F.Cu) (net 17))
 (segment (start 166.497 83.82) (end 165.862 84.455) (width 0.25) (layer F.Cu) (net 17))
 (segment (start 164.338 89.535) (end 165.862 88.011) (width 0.25) (layer F.Cu) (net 17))
 (segment (start 170.18 86.36) (end 175.26 86.36) (width 0.25) (layer F.Cu) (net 18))
 (segment (start 165.012311 89.82831) (end 164.035621 90.805) (width 0.25) (layer F.Cu) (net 18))
 (segment (start 164.035621 90.805) (end 163.56 90.805) (width 0.25) (layer F.Cu) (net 18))
 (segment (start 167.513 86.487) (end 167.64 86.36) (width 0.25) (layer F.Cu) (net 18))
 (segment (start 165.012311 89.82831) (end 166.751 88.089621) (width 0.25) (layer F.Cu) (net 18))
 (segment (start 166.751 88.089621) (end 166.751 87.249) (width 0.25) (layer F.Cu) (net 18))
 (segment (start 167.513 86.487) (end 166.751 87.249) (width 0.25) (layer F.Cu) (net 18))
 (segment (start 167.64 86.36) (end 170.18 86.36) (width 0.25) (layer F.Cu) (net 18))
 (segment (start 175.26 88.9) (end 170.18 88.9) (width 0.25) (layer F.Cu) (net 19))
 (segment (start 164.592 91.44) (end 163.957 92.075) (width 0.25) (layer F.Cu) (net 19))
 (segment (start 163.957 92.075) (end 163.56 92.075) (width 0.25) (layer F.Cu) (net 19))
 (segment (start 170.18 88.9) (end 167.64 88.9) (width 0.25) (layer F.Cu) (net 19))
 (segment (start 167.132 88.9) (end 167.64 88.9) (width 0.25) (layer F.Cu) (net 19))
 (segment (start 164.592 91.44) (end 165.608 90.424) (width 0.25) (layer F.Cu) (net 19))
 (segment (start 165.608 90.424) (end 167.132 88.9) (width 0.25) (layer F.Cu) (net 19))
 (segment (start 170.18 91.44) (end 175.26 91.44) (width 0.25) (layer F.Cu) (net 20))
 (segment (start 164.592 92.837) (end 164.084 93.345) (width 0.25) (layer F.Cu) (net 20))
 (segment (start 164.084 93.345) (end 163.56 93.345) (width 0.25) (layer F.Cu) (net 20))
 (segment (start 165.989 91.44) (end 164.592 92.837) (width 0.25) (layer F.Cu) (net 20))
 (segment (start 170.18 91.44) (end 165.989 91.44) (width 0.25) (layer F.Cu) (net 20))
 (segment (start 175.26 93.98) (end 170.18 93.98) (width 0.25) (layer F.Cu) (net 21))
 (segment (start 167.132 94.615) (end 167.767 93.98) (width 0.25) (layer F.Cu) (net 21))
 (segment (start 163.56 94.615) (end 167.132 94.615) (width 0.25) (layer F.Cu) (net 21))
 (segment (start 167.767 93.98) (end 170.18 93.98) (width 0.25) (layer F.Cu) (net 21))
 (segment (start 170.18 96.52) (end 175.26 96.52) (width 0.25) (layer F.Cu) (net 22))
 (segment (start 167.64 95.885) (end 168.275 96.52) (width 0.25) (layer F.Cu) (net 22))
 (segment (start 163.56 95.885) (end 167.64 95.885) (width 0.25) (layer F.Cu) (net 22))
 (segment (start 168.275 96.52) (end 170.18 96.52) (width 0.25) (layer F.Cu) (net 22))
 (segment (start 175.26 99.06) (end 170.18 99.06) (width 0.25) (layer F.Cu) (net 23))
 (segment (start 167.386 97.155) (end 169.291 99.06) (width 0.25) (layer F.Cu) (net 23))
 (segment (start 163.56 97.155) (end 167.386 97.155) (width 0.25) (layer F.Cu) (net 23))
 (segment (start 169.291 99.06) (end 170.18 99.06) (width 0.25) (layer F.Cu) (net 23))
 (segment (start 170.18 101.6) (end 175.26 101.6) (width 0.25) (layer F.Cu) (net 24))
 (segment (start 168.148 100.965) (end 168.783 101.6) (width 0.25) (layer F.Cu) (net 24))
 (segment (start 168.148 99.441) (end 168.148 100.965) (width 0.25) (layer F.Cu) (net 24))
 (segment (start 163.56 98.425) (end 167.132 98.425) (width 0.25) (layer F.Cu) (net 24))
 (segment (start 167.132 98.425) (end 168.148 99.441) (width 0.25) (layer F.Cu) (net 24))
 (segment (start 168.783 101.6) (end 170.18 101.6) (width 0.25) (layer F.Cu) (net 24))
 (segment (start 175.26 104.14) (end 170.18 104.14) (width 0.25) (layer F.Cu) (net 25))
 (segment (start 167.386 102.743) (end 168.783 104.14) (width 0.25) (layer F.Cu) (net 25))
 (segment (start 167.386 100.076) (end 167.386 102.743) (width 0.25) (layer F.Cu) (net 25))
 (segment (start 163.56 99.695) (end 167.005 99.695) (width 0.25) (layer F.Cu) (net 25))
 (segment (start 167.005 99.695) (end 167.386 100.076) (width 0.25) (layer F.Cu) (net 25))
 (segment (start 168.783 104.14) (end 170.18 104.14) (width 0.25) (layer F.Cu) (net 25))
 (segment (start 170.18 106.68) (end 175.26 106.68) (width 0.25) (layer F.Cu) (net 26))
 (segment (start 167.894 106.172) (end 168.402 106.68) (width 0.25) (layer F.Cu) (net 26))
 (segment (start 167.894 104.394) (end 167.894 106.172) (width 0.25) (layer F.Cu) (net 26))
 (segment (start 166.116 100.965) (end 166.624 101.473) (width 0.25) (layer F.Cu) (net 26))
 (segment (start 163.56 100.965) (end 166.116 100.965) (width 0.25) (layer F.Cu) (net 26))
 (segment (start 166.624 101.473) (end 166.624 103.124) (width 0.25) (layer F.Cu) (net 26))
 (segment (start 166.624 103.124) (end 167.894 104.394) (width 0.25) (layer F.Cu) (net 26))
 (segment (start 168.402 106.68) (end 170.18 106.68) (width 0.25) (layer F.Cu) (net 26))
 (segment (start 170.18 109.22) (end 175.26 109.22) (width 0.25) (layer F.Cu) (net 27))
 (segment (start 167.132 107.061) (end 169.291 109.22) (width 0.25) (layer F.Cu) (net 27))
 (segment (start 167.132 105.029) (end 167.132 107.061) (width 0.25) (layer F.Cu) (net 27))
 (segment (start 165.608 102.235) (end 165.862 102.489) (width 0.25) (layer F.Cu) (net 27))
 (segment (start 163.56 102.235) (end 165.608 102.235) (width 0.25) (layer F.Cu) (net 27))
 (segment (start 165.862 102.489) (end 165.862 103.759) (width 0.25) (layer F.Cu) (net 27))
 (segment (start 165.862 103.759) (end 167.132 105.029) (width 0.25) (layer F.Cu) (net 27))
 (segment (start 169.291 109.22) (end 170.18 109.22) (width 0.25) (layer F.Cu) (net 27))
 (segment (start 168.021 111.252) (end 168.529 111.76) (width 0.25) (layer F.Cu) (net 28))
 (segment (start 168.021 109.22) (end 168.021 111.252) (width 0.25) (layer F.Cu) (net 28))
 (segment (start 166.37 107.569) (end 166.37 106.172) (width 0.25) (layer F.Cu) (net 28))
 (segment (start 166.37 105.283) (end 166.37 106.172) (width 0.25) (layer F.Cu) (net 28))
 (segment (start 163.56 103.505) (end 164.592 103.505) (width 0.25) (layer F.Cu) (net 28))
 (segment (start 164.592 103.505) (end 166.37 105.283) (width 0.25) (layer F.Cu) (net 28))
 (segment (start 166.37 107.569) (end 168.021 109.22) (width 0.25) (layer F.Cu) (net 28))
 (segment (start 168.529 111.76) (end 170.18 111.76) (width 0.25) (layer F.Cu) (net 28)))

